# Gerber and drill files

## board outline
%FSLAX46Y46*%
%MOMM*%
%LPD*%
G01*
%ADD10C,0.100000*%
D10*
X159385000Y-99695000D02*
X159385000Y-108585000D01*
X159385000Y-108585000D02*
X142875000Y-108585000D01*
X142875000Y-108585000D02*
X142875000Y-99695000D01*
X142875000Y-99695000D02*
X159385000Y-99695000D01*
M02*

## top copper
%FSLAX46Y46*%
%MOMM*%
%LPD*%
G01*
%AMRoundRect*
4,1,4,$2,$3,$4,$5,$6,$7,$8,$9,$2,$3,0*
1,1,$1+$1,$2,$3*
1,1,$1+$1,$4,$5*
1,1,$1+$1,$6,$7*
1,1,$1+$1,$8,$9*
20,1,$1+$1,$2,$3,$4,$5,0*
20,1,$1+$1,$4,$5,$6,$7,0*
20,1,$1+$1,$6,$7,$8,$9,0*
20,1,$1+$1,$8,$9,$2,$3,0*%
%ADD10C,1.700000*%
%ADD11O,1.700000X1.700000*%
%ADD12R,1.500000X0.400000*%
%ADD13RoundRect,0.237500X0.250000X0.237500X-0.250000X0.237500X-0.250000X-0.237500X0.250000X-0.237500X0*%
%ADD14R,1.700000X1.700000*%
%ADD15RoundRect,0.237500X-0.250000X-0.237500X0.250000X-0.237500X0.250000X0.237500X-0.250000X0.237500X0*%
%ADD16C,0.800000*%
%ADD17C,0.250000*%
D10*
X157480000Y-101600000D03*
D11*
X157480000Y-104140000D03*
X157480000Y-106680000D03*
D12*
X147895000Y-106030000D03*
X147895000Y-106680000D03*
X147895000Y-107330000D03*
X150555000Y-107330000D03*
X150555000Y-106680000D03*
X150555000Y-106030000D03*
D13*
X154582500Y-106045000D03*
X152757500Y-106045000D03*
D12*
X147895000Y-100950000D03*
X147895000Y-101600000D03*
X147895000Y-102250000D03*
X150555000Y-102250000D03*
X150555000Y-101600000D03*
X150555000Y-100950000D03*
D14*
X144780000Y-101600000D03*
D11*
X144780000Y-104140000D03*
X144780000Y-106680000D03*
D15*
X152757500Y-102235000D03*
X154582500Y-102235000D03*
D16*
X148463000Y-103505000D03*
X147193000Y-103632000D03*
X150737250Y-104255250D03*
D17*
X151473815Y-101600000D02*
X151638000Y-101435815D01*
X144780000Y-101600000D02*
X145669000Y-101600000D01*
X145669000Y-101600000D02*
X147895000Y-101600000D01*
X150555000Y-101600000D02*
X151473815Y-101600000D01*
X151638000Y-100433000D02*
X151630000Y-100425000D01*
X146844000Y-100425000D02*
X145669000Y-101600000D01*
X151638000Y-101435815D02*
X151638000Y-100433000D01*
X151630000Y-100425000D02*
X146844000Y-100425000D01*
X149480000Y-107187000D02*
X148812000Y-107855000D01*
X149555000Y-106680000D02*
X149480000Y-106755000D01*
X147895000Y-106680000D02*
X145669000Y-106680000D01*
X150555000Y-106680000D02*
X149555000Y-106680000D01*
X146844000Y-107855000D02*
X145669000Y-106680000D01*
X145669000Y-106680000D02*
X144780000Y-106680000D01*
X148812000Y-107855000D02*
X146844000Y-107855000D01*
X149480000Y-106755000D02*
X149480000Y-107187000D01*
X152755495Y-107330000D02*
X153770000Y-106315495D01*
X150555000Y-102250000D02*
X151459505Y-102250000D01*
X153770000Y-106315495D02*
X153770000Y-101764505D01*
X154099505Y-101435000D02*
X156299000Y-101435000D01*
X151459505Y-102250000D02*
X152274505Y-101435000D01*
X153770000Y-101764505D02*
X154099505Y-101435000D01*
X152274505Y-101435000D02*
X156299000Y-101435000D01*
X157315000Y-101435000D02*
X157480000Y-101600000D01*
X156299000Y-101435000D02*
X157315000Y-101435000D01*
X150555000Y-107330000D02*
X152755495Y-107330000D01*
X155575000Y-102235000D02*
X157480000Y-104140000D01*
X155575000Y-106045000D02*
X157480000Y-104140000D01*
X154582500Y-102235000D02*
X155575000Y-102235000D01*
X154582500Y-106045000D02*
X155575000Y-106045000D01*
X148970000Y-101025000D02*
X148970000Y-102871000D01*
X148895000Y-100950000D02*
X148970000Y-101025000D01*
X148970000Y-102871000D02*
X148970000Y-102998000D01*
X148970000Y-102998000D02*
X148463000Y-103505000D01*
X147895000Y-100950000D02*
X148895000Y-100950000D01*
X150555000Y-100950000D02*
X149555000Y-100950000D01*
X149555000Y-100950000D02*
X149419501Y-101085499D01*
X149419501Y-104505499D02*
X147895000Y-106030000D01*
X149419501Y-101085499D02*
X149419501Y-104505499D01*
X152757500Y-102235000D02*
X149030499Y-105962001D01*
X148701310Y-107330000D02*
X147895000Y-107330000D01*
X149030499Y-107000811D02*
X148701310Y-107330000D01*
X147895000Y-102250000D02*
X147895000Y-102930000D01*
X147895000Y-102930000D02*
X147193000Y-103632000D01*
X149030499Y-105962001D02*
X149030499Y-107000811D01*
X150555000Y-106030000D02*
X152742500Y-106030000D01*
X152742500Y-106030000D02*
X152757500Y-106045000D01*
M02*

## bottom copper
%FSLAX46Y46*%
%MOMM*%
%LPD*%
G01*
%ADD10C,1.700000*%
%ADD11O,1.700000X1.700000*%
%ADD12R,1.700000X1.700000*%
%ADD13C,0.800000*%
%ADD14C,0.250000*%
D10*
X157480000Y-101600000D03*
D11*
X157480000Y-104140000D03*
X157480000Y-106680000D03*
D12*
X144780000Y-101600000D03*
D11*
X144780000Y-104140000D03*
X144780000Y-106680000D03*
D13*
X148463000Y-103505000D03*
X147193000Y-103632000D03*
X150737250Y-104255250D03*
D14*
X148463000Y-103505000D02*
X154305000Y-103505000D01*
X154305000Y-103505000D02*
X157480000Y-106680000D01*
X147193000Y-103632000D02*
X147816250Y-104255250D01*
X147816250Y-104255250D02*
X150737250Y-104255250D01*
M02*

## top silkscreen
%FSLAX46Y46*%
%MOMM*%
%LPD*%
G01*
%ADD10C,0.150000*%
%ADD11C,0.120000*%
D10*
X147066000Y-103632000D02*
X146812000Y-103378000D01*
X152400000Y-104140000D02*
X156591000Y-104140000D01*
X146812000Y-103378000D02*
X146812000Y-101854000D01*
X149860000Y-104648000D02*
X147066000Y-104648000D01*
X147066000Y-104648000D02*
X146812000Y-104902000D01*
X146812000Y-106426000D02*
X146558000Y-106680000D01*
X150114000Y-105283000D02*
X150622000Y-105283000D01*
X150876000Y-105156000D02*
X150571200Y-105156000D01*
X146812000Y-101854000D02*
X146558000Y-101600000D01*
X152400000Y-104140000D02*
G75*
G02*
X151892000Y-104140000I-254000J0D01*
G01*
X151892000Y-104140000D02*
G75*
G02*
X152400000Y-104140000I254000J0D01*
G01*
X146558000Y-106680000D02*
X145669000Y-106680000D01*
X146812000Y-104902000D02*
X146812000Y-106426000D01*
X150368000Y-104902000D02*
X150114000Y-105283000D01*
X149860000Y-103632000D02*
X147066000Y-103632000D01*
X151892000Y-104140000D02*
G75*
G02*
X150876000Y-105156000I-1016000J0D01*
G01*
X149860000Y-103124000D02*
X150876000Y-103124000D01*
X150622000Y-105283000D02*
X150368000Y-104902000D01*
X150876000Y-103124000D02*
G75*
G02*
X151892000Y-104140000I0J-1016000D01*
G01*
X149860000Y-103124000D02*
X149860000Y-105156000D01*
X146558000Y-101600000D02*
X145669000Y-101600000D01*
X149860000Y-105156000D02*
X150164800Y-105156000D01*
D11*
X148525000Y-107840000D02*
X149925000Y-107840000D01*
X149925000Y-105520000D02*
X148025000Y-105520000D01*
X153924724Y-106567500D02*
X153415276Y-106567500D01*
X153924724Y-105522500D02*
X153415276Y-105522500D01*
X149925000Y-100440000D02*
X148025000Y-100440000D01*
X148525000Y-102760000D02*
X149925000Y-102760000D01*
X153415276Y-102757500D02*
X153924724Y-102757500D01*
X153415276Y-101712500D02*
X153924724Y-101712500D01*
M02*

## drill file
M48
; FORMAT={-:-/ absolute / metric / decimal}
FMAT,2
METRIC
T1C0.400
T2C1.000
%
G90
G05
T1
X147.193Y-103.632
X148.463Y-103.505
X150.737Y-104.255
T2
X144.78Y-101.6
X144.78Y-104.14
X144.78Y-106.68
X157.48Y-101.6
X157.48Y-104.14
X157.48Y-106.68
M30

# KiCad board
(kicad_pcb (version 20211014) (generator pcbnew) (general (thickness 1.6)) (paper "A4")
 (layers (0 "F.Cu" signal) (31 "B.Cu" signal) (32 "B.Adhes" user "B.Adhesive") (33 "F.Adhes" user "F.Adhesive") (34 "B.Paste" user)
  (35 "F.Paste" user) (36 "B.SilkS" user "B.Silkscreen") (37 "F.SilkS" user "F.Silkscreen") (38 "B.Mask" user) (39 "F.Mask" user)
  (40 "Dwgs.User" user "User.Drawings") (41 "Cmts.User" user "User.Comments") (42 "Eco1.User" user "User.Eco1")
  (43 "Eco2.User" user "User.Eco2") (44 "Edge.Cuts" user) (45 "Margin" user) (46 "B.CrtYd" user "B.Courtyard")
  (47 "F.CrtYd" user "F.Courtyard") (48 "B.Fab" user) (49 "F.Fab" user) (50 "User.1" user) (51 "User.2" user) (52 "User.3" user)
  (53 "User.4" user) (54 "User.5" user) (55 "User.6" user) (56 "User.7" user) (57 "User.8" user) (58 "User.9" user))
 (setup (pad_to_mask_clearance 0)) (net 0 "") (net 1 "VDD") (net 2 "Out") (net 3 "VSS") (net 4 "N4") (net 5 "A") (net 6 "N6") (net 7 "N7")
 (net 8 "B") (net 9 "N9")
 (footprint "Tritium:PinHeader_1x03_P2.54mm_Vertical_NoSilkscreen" (layer "F.Cu") (at 157.48 101.6)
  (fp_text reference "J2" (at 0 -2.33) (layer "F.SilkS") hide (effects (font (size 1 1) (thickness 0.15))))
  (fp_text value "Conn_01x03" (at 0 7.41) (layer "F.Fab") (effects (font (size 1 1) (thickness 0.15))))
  (pad "1" thru_hole circle (at 0 0) (size 1.7 1.7) (drill 1) (layers *.Cu *.Mask) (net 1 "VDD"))
  (pad "2" thru_hole oval (at 0 2.54) (size 1.7 1.7) (drill 1) (layers *.Cu *.Mask) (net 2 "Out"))
  (pad "3" thru_hole oval (at 0 5.08) (size 1.7 1.7) (drill 1) (layers *.Cu *.Mask) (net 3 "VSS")))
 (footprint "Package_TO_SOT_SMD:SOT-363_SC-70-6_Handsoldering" (layer "F.Cu") (at 149.225 106.68)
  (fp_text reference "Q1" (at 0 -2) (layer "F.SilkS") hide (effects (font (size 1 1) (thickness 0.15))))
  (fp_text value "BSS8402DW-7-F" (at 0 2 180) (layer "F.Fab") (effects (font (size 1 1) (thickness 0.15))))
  (fp_line (start -0.7 1.16) (end 0.7 1.16) (layer "F.SilkS") (width 0.12))
  (fp_line (start 0.7 -1.16) (end -1.2 -1.16) (layer "F.SilkS") (width 0.12))
  (pad "1" smd rect (at -1.33 -0.65) (size 1.5 0.4) (layers "F.Cu" "F.Paste" "F.Mask") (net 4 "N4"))
  (pad "2" smd rect (at -1.33 0) (size 1.5 0.4) (layers "F.Cu" "F.Paste" "F.Mask") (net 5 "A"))
  (pad "3" smd rect (at -1.33 0.65) (size 1.5 0.4) (layers "F.Cu" "F.Paste" "F.Mask") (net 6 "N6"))
  (pad "4" smd rect (at 1.33 0.65) (size 1.5 0.4) (layers "F.Cu" "F.Paste" "F.Mask") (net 1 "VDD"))
  (pad "5" smd rect (at 1.33 0) (size 1.5 0.4) (layers "F.Cu" "F.Paste" "F.Mask") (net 5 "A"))
  (pad "6" smd rect (at 1.33 -0.65) (size 1.5 0.4) (layers "F.Cu" "F.Paste" "F.Mask") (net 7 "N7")))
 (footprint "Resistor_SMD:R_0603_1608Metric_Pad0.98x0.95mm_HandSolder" (layer "F.Cu") (at 153.67 106.045 180)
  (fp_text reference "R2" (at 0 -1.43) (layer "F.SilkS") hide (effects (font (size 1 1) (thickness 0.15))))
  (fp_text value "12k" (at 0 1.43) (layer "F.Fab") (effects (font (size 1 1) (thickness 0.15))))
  (fp_line (start -0.254724 -0.5225) (end 0.254724 -0.5225) (layer "F.SilkS") (width 0.12))
  (fp_line (start -0.254724 0.5225) (end 0.254724 0.5225) (layer "F.SilkS") (width 0.12))
  (pad "1" smd roundrect (at -0.9125 0 180) (size 0.975 0.95) (layers "F.Cu" "F.Paste" "F.Mask") (roundrect_rratio 0.25) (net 2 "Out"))
  (pad "2" smd roundrect (at 0.9125 0 180) (size 0.975 0.95) (layers "F.Cu" "F.Paste" "F.Mask") (roundrect_rratio 0.25) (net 7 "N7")))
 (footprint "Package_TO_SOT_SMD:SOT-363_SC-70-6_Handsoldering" (layer "F.Cu") (at 149.225 101.6)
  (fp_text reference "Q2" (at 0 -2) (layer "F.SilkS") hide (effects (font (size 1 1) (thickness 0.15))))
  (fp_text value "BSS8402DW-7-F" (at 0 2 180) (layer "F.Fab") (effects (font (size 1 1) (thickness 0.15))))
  (fp_line (start 0.7 -1.16) (end -1.2 -1.16) (layer "F.SilkS") (width 0.12))
  (fp_line (start -0.7 1.16) (end 0.7 1.16) (layer "F.SilkS") (width 0.12))
  (pad "1" smd rect (at -1.33 -0.65) (size 1.5 0.4) (layers "F.Cu" "F.Paste" "F.Mask") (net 3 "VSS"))
  (pad "2" smd rect (at -1.33 0) (size 1.5 0.4) (layers "F.Cu" "F.Paste" "F.Mask") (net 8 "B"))
  (pad "3" smd rect (at -1.33 0.65) (size 1.5 0.4) (layers "F.Cu" "F.Paste" "F.Mask") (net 6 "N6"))
  (pad "4" smd rect (at 1.33 0.65) (size 1.5 0.4) (layers "F.Cu" "F.Paste" "F.Mask") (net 1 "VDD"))
  (pad "5" smd rect (at 1.33 0) (size 1.5 0.4) (layers "F.Cu" "F.Paste" "F.Mask") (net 8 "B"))
  (pad "6" smd rect (at 1.33 -0.65) (size 1.5 0.4) (layers "F.Cu" "F.Paste" "F.Mask") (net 4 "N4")))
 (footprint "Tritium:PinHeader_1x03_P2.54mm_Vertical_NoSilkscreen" (layer "F.Cu") (at 144.78 101.6)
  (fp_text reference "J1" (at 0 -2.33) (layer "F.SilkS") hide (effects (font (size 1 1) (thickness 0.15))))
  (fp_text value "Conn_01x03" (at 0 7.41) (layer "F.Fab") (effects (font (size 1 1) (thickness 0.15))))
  (pad "1" thru_hole rect (at 0 0) (size 1.7 1.7) (drill 1) (layers *.Cu *.Mask) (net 8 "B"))
  (pad "2" thru_hole oval (at 0 2.54) (size 1.7 1.7) (drill 1) (layers *.Cu *.Mask) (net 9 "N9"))
  (pad "3" thru_hole oval (at 0 5.08) (size 1.7 1.7) (drill 1) (layers *.Cu *.Mask) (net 5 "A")))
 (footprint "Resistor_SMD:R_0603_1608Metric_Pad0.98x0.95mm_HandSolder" (layer "F.Cu") (at 153.67 102.235)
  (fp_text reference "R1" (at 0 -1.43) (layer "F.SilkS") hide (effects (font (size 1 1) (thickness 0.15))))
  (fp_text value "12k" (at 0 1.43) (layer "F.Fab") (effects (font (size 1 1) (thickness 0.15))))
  (fp_line (start -0.254724 0.5225) (end 0.254724 0.5225) (layer "F.SilkS") (width 0.12))
  (fp_line (start -0.254724 -0.5225) (end 0.254724 -0.5225) (layer "F.SilkS") (width 0.12))
  (pad "1" smd roundrect (at -0.9125 0) (size 0.975 0.95) (layers "F.Cu" "F.Paste" "F.Mask") (roundrect_rratio 0.25) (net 6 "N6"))
  (pad "2" smd roundrect (at 0.9125 0) (size 0.975 0.95) (layers "F.Cu" "F.Paste" "F.Mask") (roundrect_rratio 0.25) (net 2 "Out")))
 (gr_line (start 147.066 103.632) (end 146.812 103.378) (layer "F.SilkS") (width 0.15))
 (gr_line (start 152.4 104.14) (end 156.591 104.14) (layer "F.SilkS") (width 0.15))
 (gr_line (start 146.812 103.378) (end 146.812 101.854) (layer "F.SilkS") (width 0.15))
 (gr_line (start 149.86 104.648) (end 147.066 104.648) (layer "F.SilkS") (width 0.15))
 (gr_line (start 147.066 104.648) (end 146.812 104.902) (layer "F.SilkS") (width 0.15))
 (gr_line (start 146.812 106.426) (end 146.558 106.68) (layer "F.SilkS") (width 0.15))
 (gr_line (start 150.114 105.283) (end 150.622 105.283) (layer "F.SilkS") (width 0.15))
 (gr_line (start 150.876 105.156) (end 150.5712 105.156) (layer "F.SilkS") (width 0.15))
 (gr_line (start 146.812 101.854) (end 146.558 101.6) (layer "F.SilkS") (width 0.15))
 (gr_circle (center 152.146 104.14) (end 152.4 104.14) (layer "F.SilkS") (width 0.15) (fill none))
 (gr_line (start 146.558 106.68) (end 145.669 106.68) (layer "F.SilkS") (width 0.15))
 (gr_line (start 146.812 104.902) (end 146.812 106.426) (layer "F.SilkS") (width 0.15))
 (gr_line (start 150.368 104.902) (end 150.114 105.283) (layer "F.SilkS") (width 0.15))
 (gr_line (start 149.86 103.632) (end 147.066 103.632) (layer "F.SilkS") (width 0.15))
 (gr_arc (start 151.892 104.14) (mid 151.59442 104.85842) (end 150.876 105.156) (layer "F.SilkS") (width 0.15))
 (gr_line (start 149.86 103.124) (end 150.876 103.124) (layer "F.SilkS") (width 0.15))
 (gr_line (start 150.622 105.283) (end 150.368 104.902) (layer "F.SilkS") (width 0.15))
 (gr_arc (start 150.876 103.124) (mid 151.59442 103.42158) (end 151.892 104.14) (layer "F.SilkS") (width 0.15))
 (gr_line (start 149.86 103.124) (end 149.86 105.156) (layer "F.SilkS") (width 0.15))
 (gr_line (start 146.558 101.6) (end 145.669 101.6) (layer "F.SilkS") (width 0.15))
 (gr_line (start 149.86 105.156) (end 150.1648 105.156) (layer "F.SilkS") (width 0.15))
 (gr_line (start 159.385 99.695) (end 159.385 108.585) (layer "Edge.Cuts") (width 0.1))
 (gr_line (start 159.385 108.585) (end 142.875 108.585) (layer "Edge.Cuts") (width 0.1))
 (gr_line (start 142.875 108.585) (end 142.875 99.695) (layer "Edge.Cuts") (width 0.1))
 (gr_line (start 142.875 99.695) (end 159.385 99.695) (layer "Edge.Cuts") (width 0.1))
 (segment (start 151.473815 101.6) (end 151.638 101.435815) (width 0.25) (layer "F.Cu") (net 8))
 (segment (start 144.78 101.6) (end 145.669 101.6) (width 0.25) (layer "F.Cu") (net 8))
 (segment (start 145.669 101.6) (end 147.895 101.6) (width 0.25) (layer "F.Cu") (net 8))
 (segment (start 150.555 101.6) (end 151.473815 101.6) (width 0.25) (layer "F.Cu") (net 8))
 (segment (start 151.638 100.433) (end 151.63 100.425) (width 0.25) (layer "F.Cu") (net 8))
 (segment (start 146.844 100.425) (end 145.669 101.6) (width 0.25) (layer "F.Cu") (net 8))
 (segment (start 151.638 101.435815) (end 151.638 100.433) (width 0.25) (layer "F.Cu") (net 8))
 (segment (start 151.63 100.425) (end 146.844 100.425) (width 0.25) (layer "F.Cu") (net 8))
 (segment (start 149.48 107.187) (end 148.812 107.855) (width 0.25) (layer "F.Cu") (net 5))
 (segment (start 149.555 106.68) (end 149.48 106.755) (width 0.25) (layer "F.Cu") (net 5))
 (segment (start 147.895 106.68) (end 145.669 106.68) (width 0.25) (layer "F.Cu") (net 5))
 (segment (start 150.555 106.68) (end 149.555 106.68) (width 0.25) (layer "F.Cu") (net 5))
 (segment (start 146.844 107.855) (end 145.669 106.68) (width 0.25) (layer "F.Cu") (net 5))
 (segment (start 145.669 106.68) (end 144.78 106.68) (width 0.25) (layer "F.Cu") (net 5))
 (segment (start 148.812 107.855) (end 146.844 107.855) (width 0.25) (layer "F.Cu") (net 5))
 (segment (start 149.48 106.755) (end 149.48 107.187) (width 0.25) (layer "F.Cu") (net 5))
 (segment (start 152.755495 107.33) (end 153.77 106.315495) (width 0.25) (layer "F.Cu") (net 1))
 (segment (start 150.555 102.25) (end 151.459505 102.25) (width 0.25) (layer "F.Cu") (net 1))
 (segment (start 153.77 106.315495) (end 153.77 101.764505) (width 0.25) (layer "F.Cu") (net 1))
 (segment (start 154.099505 101.435) (end 156.299 101.435) (width 0.25) (layer "F.Cu") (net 1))
 (segment (start 151.459505 102.25) (end 152.274505 101.435) (width 0.25) (layer "F.Cu") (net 1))
 (segment (start 153.77 101.764505) (end 154.099505 101.435) (width 0.25) (layer "F.Cu") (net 1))
 (segment (start 152.274505 101.435) (end 156.299 101.435) (width 0.25) (layer "F.Cu") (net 1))
 (segment (start 157.315 101.435) (end 157.48 101.6) (width 0.25) (layer "F.Cu") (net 1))
 (segment (start 156.299 101.435) (end 157.315 101.435) (width 0.25) (layer "F.Cu") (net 1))
 (segment (start 150.555 107.33) (end 152.755495 107.33) (width 0.25) (layer "F.Cu") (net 1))
 (segment (start 155.575 102.235) (end 157.48 104.14) (width 0.25) (layer "F.Cu") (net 2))
 (segment (start 155.575 106.045) (end 157.48 104.14) (width 0.25) (layer "F.Cu") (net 2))
 (segment (start 154.5825 102.235) (end 155.575 102.235) (width 0.25) (layer "F.Cu") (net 2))
 (segment (start 154.5825 106.045) (end 155.575 106.045) (width 0.25) (layer "F.Cu") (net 2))
 (segment (start 148.97 101.025) (end 148.97 102.871) (width 0.25) (layer "F.Cu") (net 3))
 (segment (start 148.895 100.95) (end 148.97 101.025) (width 0.25) (layer "F.Cu") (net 3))
 (segment (start 148.97 102.871) (end 148.97 102.998) (width 0.25) (layer "F.Cu") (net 3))
 (segment (start 148.97 102.998) (end 148.463 103.505) (width 0.25) (layer "F.Cu") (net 3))
 (segment (start 147.895 100.95) (end 148.895 100.95) (width 0.25) (layer "F.Cu") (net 3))
 (via (at 148.463 103.505) (size 0.8) (drill 0.4) (layers "F.Cu" "B.Cu") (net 3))
 (segment (start 148.463 103.505) (end 154.305 103.505) (width 0.25) (layer "B.Cu") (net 3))
 (segment (start 154.305 103.505) (end 157.48 106.68) (width 0.25) (layer "B.Cu") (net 3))
 (segment (start 150.555 100.95) (end 149.555 100.95) (width 0.25) (layer "F.Cu") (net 4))
 (segment (start 149.555 100.95) (end 149.419501 101.085499) (width 0.25) (layer "F.Cu") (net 4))
 (segment (start 149.419501 104.505499) (end 147.895 106.03) (width 0.25) (layer "F.Cu") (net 4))
 (segment (start 149.419501 101.085499) (end 149.419501 104.505499) (width 0.25) (layer "F.Cu") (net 4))
 (segment (start 152.7575 102.235) (end 149.030499 105.962001) (width 0.25) (layer "F.Cu") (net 6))
 (segment (start 148.70131 107.33) (end 147.895 107.33) (width 0.25) (layer "F.Cu") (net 6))
 (segment (start 149.030499 107.000811) (end 148.70131 107.33) (width 0.25) (layer "F.Cu") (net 6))
 (segment (start 147.895 102.25) (end 147.895 102.93) (width 0.25) (layer "F.Cu") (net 6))
 (segment (start 147.895 102.93) (end 147.193 103.632) (width 0.25) (layer "F.Cu") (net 6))
 (segment (start 149.030499 105.962001) (end 149.030499 107.000811) (width 0.25) (layer "F.Cu") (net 6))
 (via (at 147.193 103.632) (size 0.8) (drill 0.4) (layers "F.Cu" "B.Cu") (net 6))
 (via (at 150.73725 104.25525) (size 0.8) (drill 0.4) (layers "F.Cu" "B.Cu") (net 6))
 (segment (start 147.193 103.632) (end 147.81625 104.25525) (width 0.25) (layer "B.Cu") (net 6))
 (segment (start 147.81625 104.25525) (end 150.73725 104.25525) (width 0.25) (layer "B.Cu") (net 6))
 (segment (start 150.555 106.03) (end 152.7425 106.03) (width 0.25) (layer "F.Cu") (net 7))
 (segment (start 152.7425 106.03) (end 152.7575 106.045) (width 0.25) (layer "F.Cu") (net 7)))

